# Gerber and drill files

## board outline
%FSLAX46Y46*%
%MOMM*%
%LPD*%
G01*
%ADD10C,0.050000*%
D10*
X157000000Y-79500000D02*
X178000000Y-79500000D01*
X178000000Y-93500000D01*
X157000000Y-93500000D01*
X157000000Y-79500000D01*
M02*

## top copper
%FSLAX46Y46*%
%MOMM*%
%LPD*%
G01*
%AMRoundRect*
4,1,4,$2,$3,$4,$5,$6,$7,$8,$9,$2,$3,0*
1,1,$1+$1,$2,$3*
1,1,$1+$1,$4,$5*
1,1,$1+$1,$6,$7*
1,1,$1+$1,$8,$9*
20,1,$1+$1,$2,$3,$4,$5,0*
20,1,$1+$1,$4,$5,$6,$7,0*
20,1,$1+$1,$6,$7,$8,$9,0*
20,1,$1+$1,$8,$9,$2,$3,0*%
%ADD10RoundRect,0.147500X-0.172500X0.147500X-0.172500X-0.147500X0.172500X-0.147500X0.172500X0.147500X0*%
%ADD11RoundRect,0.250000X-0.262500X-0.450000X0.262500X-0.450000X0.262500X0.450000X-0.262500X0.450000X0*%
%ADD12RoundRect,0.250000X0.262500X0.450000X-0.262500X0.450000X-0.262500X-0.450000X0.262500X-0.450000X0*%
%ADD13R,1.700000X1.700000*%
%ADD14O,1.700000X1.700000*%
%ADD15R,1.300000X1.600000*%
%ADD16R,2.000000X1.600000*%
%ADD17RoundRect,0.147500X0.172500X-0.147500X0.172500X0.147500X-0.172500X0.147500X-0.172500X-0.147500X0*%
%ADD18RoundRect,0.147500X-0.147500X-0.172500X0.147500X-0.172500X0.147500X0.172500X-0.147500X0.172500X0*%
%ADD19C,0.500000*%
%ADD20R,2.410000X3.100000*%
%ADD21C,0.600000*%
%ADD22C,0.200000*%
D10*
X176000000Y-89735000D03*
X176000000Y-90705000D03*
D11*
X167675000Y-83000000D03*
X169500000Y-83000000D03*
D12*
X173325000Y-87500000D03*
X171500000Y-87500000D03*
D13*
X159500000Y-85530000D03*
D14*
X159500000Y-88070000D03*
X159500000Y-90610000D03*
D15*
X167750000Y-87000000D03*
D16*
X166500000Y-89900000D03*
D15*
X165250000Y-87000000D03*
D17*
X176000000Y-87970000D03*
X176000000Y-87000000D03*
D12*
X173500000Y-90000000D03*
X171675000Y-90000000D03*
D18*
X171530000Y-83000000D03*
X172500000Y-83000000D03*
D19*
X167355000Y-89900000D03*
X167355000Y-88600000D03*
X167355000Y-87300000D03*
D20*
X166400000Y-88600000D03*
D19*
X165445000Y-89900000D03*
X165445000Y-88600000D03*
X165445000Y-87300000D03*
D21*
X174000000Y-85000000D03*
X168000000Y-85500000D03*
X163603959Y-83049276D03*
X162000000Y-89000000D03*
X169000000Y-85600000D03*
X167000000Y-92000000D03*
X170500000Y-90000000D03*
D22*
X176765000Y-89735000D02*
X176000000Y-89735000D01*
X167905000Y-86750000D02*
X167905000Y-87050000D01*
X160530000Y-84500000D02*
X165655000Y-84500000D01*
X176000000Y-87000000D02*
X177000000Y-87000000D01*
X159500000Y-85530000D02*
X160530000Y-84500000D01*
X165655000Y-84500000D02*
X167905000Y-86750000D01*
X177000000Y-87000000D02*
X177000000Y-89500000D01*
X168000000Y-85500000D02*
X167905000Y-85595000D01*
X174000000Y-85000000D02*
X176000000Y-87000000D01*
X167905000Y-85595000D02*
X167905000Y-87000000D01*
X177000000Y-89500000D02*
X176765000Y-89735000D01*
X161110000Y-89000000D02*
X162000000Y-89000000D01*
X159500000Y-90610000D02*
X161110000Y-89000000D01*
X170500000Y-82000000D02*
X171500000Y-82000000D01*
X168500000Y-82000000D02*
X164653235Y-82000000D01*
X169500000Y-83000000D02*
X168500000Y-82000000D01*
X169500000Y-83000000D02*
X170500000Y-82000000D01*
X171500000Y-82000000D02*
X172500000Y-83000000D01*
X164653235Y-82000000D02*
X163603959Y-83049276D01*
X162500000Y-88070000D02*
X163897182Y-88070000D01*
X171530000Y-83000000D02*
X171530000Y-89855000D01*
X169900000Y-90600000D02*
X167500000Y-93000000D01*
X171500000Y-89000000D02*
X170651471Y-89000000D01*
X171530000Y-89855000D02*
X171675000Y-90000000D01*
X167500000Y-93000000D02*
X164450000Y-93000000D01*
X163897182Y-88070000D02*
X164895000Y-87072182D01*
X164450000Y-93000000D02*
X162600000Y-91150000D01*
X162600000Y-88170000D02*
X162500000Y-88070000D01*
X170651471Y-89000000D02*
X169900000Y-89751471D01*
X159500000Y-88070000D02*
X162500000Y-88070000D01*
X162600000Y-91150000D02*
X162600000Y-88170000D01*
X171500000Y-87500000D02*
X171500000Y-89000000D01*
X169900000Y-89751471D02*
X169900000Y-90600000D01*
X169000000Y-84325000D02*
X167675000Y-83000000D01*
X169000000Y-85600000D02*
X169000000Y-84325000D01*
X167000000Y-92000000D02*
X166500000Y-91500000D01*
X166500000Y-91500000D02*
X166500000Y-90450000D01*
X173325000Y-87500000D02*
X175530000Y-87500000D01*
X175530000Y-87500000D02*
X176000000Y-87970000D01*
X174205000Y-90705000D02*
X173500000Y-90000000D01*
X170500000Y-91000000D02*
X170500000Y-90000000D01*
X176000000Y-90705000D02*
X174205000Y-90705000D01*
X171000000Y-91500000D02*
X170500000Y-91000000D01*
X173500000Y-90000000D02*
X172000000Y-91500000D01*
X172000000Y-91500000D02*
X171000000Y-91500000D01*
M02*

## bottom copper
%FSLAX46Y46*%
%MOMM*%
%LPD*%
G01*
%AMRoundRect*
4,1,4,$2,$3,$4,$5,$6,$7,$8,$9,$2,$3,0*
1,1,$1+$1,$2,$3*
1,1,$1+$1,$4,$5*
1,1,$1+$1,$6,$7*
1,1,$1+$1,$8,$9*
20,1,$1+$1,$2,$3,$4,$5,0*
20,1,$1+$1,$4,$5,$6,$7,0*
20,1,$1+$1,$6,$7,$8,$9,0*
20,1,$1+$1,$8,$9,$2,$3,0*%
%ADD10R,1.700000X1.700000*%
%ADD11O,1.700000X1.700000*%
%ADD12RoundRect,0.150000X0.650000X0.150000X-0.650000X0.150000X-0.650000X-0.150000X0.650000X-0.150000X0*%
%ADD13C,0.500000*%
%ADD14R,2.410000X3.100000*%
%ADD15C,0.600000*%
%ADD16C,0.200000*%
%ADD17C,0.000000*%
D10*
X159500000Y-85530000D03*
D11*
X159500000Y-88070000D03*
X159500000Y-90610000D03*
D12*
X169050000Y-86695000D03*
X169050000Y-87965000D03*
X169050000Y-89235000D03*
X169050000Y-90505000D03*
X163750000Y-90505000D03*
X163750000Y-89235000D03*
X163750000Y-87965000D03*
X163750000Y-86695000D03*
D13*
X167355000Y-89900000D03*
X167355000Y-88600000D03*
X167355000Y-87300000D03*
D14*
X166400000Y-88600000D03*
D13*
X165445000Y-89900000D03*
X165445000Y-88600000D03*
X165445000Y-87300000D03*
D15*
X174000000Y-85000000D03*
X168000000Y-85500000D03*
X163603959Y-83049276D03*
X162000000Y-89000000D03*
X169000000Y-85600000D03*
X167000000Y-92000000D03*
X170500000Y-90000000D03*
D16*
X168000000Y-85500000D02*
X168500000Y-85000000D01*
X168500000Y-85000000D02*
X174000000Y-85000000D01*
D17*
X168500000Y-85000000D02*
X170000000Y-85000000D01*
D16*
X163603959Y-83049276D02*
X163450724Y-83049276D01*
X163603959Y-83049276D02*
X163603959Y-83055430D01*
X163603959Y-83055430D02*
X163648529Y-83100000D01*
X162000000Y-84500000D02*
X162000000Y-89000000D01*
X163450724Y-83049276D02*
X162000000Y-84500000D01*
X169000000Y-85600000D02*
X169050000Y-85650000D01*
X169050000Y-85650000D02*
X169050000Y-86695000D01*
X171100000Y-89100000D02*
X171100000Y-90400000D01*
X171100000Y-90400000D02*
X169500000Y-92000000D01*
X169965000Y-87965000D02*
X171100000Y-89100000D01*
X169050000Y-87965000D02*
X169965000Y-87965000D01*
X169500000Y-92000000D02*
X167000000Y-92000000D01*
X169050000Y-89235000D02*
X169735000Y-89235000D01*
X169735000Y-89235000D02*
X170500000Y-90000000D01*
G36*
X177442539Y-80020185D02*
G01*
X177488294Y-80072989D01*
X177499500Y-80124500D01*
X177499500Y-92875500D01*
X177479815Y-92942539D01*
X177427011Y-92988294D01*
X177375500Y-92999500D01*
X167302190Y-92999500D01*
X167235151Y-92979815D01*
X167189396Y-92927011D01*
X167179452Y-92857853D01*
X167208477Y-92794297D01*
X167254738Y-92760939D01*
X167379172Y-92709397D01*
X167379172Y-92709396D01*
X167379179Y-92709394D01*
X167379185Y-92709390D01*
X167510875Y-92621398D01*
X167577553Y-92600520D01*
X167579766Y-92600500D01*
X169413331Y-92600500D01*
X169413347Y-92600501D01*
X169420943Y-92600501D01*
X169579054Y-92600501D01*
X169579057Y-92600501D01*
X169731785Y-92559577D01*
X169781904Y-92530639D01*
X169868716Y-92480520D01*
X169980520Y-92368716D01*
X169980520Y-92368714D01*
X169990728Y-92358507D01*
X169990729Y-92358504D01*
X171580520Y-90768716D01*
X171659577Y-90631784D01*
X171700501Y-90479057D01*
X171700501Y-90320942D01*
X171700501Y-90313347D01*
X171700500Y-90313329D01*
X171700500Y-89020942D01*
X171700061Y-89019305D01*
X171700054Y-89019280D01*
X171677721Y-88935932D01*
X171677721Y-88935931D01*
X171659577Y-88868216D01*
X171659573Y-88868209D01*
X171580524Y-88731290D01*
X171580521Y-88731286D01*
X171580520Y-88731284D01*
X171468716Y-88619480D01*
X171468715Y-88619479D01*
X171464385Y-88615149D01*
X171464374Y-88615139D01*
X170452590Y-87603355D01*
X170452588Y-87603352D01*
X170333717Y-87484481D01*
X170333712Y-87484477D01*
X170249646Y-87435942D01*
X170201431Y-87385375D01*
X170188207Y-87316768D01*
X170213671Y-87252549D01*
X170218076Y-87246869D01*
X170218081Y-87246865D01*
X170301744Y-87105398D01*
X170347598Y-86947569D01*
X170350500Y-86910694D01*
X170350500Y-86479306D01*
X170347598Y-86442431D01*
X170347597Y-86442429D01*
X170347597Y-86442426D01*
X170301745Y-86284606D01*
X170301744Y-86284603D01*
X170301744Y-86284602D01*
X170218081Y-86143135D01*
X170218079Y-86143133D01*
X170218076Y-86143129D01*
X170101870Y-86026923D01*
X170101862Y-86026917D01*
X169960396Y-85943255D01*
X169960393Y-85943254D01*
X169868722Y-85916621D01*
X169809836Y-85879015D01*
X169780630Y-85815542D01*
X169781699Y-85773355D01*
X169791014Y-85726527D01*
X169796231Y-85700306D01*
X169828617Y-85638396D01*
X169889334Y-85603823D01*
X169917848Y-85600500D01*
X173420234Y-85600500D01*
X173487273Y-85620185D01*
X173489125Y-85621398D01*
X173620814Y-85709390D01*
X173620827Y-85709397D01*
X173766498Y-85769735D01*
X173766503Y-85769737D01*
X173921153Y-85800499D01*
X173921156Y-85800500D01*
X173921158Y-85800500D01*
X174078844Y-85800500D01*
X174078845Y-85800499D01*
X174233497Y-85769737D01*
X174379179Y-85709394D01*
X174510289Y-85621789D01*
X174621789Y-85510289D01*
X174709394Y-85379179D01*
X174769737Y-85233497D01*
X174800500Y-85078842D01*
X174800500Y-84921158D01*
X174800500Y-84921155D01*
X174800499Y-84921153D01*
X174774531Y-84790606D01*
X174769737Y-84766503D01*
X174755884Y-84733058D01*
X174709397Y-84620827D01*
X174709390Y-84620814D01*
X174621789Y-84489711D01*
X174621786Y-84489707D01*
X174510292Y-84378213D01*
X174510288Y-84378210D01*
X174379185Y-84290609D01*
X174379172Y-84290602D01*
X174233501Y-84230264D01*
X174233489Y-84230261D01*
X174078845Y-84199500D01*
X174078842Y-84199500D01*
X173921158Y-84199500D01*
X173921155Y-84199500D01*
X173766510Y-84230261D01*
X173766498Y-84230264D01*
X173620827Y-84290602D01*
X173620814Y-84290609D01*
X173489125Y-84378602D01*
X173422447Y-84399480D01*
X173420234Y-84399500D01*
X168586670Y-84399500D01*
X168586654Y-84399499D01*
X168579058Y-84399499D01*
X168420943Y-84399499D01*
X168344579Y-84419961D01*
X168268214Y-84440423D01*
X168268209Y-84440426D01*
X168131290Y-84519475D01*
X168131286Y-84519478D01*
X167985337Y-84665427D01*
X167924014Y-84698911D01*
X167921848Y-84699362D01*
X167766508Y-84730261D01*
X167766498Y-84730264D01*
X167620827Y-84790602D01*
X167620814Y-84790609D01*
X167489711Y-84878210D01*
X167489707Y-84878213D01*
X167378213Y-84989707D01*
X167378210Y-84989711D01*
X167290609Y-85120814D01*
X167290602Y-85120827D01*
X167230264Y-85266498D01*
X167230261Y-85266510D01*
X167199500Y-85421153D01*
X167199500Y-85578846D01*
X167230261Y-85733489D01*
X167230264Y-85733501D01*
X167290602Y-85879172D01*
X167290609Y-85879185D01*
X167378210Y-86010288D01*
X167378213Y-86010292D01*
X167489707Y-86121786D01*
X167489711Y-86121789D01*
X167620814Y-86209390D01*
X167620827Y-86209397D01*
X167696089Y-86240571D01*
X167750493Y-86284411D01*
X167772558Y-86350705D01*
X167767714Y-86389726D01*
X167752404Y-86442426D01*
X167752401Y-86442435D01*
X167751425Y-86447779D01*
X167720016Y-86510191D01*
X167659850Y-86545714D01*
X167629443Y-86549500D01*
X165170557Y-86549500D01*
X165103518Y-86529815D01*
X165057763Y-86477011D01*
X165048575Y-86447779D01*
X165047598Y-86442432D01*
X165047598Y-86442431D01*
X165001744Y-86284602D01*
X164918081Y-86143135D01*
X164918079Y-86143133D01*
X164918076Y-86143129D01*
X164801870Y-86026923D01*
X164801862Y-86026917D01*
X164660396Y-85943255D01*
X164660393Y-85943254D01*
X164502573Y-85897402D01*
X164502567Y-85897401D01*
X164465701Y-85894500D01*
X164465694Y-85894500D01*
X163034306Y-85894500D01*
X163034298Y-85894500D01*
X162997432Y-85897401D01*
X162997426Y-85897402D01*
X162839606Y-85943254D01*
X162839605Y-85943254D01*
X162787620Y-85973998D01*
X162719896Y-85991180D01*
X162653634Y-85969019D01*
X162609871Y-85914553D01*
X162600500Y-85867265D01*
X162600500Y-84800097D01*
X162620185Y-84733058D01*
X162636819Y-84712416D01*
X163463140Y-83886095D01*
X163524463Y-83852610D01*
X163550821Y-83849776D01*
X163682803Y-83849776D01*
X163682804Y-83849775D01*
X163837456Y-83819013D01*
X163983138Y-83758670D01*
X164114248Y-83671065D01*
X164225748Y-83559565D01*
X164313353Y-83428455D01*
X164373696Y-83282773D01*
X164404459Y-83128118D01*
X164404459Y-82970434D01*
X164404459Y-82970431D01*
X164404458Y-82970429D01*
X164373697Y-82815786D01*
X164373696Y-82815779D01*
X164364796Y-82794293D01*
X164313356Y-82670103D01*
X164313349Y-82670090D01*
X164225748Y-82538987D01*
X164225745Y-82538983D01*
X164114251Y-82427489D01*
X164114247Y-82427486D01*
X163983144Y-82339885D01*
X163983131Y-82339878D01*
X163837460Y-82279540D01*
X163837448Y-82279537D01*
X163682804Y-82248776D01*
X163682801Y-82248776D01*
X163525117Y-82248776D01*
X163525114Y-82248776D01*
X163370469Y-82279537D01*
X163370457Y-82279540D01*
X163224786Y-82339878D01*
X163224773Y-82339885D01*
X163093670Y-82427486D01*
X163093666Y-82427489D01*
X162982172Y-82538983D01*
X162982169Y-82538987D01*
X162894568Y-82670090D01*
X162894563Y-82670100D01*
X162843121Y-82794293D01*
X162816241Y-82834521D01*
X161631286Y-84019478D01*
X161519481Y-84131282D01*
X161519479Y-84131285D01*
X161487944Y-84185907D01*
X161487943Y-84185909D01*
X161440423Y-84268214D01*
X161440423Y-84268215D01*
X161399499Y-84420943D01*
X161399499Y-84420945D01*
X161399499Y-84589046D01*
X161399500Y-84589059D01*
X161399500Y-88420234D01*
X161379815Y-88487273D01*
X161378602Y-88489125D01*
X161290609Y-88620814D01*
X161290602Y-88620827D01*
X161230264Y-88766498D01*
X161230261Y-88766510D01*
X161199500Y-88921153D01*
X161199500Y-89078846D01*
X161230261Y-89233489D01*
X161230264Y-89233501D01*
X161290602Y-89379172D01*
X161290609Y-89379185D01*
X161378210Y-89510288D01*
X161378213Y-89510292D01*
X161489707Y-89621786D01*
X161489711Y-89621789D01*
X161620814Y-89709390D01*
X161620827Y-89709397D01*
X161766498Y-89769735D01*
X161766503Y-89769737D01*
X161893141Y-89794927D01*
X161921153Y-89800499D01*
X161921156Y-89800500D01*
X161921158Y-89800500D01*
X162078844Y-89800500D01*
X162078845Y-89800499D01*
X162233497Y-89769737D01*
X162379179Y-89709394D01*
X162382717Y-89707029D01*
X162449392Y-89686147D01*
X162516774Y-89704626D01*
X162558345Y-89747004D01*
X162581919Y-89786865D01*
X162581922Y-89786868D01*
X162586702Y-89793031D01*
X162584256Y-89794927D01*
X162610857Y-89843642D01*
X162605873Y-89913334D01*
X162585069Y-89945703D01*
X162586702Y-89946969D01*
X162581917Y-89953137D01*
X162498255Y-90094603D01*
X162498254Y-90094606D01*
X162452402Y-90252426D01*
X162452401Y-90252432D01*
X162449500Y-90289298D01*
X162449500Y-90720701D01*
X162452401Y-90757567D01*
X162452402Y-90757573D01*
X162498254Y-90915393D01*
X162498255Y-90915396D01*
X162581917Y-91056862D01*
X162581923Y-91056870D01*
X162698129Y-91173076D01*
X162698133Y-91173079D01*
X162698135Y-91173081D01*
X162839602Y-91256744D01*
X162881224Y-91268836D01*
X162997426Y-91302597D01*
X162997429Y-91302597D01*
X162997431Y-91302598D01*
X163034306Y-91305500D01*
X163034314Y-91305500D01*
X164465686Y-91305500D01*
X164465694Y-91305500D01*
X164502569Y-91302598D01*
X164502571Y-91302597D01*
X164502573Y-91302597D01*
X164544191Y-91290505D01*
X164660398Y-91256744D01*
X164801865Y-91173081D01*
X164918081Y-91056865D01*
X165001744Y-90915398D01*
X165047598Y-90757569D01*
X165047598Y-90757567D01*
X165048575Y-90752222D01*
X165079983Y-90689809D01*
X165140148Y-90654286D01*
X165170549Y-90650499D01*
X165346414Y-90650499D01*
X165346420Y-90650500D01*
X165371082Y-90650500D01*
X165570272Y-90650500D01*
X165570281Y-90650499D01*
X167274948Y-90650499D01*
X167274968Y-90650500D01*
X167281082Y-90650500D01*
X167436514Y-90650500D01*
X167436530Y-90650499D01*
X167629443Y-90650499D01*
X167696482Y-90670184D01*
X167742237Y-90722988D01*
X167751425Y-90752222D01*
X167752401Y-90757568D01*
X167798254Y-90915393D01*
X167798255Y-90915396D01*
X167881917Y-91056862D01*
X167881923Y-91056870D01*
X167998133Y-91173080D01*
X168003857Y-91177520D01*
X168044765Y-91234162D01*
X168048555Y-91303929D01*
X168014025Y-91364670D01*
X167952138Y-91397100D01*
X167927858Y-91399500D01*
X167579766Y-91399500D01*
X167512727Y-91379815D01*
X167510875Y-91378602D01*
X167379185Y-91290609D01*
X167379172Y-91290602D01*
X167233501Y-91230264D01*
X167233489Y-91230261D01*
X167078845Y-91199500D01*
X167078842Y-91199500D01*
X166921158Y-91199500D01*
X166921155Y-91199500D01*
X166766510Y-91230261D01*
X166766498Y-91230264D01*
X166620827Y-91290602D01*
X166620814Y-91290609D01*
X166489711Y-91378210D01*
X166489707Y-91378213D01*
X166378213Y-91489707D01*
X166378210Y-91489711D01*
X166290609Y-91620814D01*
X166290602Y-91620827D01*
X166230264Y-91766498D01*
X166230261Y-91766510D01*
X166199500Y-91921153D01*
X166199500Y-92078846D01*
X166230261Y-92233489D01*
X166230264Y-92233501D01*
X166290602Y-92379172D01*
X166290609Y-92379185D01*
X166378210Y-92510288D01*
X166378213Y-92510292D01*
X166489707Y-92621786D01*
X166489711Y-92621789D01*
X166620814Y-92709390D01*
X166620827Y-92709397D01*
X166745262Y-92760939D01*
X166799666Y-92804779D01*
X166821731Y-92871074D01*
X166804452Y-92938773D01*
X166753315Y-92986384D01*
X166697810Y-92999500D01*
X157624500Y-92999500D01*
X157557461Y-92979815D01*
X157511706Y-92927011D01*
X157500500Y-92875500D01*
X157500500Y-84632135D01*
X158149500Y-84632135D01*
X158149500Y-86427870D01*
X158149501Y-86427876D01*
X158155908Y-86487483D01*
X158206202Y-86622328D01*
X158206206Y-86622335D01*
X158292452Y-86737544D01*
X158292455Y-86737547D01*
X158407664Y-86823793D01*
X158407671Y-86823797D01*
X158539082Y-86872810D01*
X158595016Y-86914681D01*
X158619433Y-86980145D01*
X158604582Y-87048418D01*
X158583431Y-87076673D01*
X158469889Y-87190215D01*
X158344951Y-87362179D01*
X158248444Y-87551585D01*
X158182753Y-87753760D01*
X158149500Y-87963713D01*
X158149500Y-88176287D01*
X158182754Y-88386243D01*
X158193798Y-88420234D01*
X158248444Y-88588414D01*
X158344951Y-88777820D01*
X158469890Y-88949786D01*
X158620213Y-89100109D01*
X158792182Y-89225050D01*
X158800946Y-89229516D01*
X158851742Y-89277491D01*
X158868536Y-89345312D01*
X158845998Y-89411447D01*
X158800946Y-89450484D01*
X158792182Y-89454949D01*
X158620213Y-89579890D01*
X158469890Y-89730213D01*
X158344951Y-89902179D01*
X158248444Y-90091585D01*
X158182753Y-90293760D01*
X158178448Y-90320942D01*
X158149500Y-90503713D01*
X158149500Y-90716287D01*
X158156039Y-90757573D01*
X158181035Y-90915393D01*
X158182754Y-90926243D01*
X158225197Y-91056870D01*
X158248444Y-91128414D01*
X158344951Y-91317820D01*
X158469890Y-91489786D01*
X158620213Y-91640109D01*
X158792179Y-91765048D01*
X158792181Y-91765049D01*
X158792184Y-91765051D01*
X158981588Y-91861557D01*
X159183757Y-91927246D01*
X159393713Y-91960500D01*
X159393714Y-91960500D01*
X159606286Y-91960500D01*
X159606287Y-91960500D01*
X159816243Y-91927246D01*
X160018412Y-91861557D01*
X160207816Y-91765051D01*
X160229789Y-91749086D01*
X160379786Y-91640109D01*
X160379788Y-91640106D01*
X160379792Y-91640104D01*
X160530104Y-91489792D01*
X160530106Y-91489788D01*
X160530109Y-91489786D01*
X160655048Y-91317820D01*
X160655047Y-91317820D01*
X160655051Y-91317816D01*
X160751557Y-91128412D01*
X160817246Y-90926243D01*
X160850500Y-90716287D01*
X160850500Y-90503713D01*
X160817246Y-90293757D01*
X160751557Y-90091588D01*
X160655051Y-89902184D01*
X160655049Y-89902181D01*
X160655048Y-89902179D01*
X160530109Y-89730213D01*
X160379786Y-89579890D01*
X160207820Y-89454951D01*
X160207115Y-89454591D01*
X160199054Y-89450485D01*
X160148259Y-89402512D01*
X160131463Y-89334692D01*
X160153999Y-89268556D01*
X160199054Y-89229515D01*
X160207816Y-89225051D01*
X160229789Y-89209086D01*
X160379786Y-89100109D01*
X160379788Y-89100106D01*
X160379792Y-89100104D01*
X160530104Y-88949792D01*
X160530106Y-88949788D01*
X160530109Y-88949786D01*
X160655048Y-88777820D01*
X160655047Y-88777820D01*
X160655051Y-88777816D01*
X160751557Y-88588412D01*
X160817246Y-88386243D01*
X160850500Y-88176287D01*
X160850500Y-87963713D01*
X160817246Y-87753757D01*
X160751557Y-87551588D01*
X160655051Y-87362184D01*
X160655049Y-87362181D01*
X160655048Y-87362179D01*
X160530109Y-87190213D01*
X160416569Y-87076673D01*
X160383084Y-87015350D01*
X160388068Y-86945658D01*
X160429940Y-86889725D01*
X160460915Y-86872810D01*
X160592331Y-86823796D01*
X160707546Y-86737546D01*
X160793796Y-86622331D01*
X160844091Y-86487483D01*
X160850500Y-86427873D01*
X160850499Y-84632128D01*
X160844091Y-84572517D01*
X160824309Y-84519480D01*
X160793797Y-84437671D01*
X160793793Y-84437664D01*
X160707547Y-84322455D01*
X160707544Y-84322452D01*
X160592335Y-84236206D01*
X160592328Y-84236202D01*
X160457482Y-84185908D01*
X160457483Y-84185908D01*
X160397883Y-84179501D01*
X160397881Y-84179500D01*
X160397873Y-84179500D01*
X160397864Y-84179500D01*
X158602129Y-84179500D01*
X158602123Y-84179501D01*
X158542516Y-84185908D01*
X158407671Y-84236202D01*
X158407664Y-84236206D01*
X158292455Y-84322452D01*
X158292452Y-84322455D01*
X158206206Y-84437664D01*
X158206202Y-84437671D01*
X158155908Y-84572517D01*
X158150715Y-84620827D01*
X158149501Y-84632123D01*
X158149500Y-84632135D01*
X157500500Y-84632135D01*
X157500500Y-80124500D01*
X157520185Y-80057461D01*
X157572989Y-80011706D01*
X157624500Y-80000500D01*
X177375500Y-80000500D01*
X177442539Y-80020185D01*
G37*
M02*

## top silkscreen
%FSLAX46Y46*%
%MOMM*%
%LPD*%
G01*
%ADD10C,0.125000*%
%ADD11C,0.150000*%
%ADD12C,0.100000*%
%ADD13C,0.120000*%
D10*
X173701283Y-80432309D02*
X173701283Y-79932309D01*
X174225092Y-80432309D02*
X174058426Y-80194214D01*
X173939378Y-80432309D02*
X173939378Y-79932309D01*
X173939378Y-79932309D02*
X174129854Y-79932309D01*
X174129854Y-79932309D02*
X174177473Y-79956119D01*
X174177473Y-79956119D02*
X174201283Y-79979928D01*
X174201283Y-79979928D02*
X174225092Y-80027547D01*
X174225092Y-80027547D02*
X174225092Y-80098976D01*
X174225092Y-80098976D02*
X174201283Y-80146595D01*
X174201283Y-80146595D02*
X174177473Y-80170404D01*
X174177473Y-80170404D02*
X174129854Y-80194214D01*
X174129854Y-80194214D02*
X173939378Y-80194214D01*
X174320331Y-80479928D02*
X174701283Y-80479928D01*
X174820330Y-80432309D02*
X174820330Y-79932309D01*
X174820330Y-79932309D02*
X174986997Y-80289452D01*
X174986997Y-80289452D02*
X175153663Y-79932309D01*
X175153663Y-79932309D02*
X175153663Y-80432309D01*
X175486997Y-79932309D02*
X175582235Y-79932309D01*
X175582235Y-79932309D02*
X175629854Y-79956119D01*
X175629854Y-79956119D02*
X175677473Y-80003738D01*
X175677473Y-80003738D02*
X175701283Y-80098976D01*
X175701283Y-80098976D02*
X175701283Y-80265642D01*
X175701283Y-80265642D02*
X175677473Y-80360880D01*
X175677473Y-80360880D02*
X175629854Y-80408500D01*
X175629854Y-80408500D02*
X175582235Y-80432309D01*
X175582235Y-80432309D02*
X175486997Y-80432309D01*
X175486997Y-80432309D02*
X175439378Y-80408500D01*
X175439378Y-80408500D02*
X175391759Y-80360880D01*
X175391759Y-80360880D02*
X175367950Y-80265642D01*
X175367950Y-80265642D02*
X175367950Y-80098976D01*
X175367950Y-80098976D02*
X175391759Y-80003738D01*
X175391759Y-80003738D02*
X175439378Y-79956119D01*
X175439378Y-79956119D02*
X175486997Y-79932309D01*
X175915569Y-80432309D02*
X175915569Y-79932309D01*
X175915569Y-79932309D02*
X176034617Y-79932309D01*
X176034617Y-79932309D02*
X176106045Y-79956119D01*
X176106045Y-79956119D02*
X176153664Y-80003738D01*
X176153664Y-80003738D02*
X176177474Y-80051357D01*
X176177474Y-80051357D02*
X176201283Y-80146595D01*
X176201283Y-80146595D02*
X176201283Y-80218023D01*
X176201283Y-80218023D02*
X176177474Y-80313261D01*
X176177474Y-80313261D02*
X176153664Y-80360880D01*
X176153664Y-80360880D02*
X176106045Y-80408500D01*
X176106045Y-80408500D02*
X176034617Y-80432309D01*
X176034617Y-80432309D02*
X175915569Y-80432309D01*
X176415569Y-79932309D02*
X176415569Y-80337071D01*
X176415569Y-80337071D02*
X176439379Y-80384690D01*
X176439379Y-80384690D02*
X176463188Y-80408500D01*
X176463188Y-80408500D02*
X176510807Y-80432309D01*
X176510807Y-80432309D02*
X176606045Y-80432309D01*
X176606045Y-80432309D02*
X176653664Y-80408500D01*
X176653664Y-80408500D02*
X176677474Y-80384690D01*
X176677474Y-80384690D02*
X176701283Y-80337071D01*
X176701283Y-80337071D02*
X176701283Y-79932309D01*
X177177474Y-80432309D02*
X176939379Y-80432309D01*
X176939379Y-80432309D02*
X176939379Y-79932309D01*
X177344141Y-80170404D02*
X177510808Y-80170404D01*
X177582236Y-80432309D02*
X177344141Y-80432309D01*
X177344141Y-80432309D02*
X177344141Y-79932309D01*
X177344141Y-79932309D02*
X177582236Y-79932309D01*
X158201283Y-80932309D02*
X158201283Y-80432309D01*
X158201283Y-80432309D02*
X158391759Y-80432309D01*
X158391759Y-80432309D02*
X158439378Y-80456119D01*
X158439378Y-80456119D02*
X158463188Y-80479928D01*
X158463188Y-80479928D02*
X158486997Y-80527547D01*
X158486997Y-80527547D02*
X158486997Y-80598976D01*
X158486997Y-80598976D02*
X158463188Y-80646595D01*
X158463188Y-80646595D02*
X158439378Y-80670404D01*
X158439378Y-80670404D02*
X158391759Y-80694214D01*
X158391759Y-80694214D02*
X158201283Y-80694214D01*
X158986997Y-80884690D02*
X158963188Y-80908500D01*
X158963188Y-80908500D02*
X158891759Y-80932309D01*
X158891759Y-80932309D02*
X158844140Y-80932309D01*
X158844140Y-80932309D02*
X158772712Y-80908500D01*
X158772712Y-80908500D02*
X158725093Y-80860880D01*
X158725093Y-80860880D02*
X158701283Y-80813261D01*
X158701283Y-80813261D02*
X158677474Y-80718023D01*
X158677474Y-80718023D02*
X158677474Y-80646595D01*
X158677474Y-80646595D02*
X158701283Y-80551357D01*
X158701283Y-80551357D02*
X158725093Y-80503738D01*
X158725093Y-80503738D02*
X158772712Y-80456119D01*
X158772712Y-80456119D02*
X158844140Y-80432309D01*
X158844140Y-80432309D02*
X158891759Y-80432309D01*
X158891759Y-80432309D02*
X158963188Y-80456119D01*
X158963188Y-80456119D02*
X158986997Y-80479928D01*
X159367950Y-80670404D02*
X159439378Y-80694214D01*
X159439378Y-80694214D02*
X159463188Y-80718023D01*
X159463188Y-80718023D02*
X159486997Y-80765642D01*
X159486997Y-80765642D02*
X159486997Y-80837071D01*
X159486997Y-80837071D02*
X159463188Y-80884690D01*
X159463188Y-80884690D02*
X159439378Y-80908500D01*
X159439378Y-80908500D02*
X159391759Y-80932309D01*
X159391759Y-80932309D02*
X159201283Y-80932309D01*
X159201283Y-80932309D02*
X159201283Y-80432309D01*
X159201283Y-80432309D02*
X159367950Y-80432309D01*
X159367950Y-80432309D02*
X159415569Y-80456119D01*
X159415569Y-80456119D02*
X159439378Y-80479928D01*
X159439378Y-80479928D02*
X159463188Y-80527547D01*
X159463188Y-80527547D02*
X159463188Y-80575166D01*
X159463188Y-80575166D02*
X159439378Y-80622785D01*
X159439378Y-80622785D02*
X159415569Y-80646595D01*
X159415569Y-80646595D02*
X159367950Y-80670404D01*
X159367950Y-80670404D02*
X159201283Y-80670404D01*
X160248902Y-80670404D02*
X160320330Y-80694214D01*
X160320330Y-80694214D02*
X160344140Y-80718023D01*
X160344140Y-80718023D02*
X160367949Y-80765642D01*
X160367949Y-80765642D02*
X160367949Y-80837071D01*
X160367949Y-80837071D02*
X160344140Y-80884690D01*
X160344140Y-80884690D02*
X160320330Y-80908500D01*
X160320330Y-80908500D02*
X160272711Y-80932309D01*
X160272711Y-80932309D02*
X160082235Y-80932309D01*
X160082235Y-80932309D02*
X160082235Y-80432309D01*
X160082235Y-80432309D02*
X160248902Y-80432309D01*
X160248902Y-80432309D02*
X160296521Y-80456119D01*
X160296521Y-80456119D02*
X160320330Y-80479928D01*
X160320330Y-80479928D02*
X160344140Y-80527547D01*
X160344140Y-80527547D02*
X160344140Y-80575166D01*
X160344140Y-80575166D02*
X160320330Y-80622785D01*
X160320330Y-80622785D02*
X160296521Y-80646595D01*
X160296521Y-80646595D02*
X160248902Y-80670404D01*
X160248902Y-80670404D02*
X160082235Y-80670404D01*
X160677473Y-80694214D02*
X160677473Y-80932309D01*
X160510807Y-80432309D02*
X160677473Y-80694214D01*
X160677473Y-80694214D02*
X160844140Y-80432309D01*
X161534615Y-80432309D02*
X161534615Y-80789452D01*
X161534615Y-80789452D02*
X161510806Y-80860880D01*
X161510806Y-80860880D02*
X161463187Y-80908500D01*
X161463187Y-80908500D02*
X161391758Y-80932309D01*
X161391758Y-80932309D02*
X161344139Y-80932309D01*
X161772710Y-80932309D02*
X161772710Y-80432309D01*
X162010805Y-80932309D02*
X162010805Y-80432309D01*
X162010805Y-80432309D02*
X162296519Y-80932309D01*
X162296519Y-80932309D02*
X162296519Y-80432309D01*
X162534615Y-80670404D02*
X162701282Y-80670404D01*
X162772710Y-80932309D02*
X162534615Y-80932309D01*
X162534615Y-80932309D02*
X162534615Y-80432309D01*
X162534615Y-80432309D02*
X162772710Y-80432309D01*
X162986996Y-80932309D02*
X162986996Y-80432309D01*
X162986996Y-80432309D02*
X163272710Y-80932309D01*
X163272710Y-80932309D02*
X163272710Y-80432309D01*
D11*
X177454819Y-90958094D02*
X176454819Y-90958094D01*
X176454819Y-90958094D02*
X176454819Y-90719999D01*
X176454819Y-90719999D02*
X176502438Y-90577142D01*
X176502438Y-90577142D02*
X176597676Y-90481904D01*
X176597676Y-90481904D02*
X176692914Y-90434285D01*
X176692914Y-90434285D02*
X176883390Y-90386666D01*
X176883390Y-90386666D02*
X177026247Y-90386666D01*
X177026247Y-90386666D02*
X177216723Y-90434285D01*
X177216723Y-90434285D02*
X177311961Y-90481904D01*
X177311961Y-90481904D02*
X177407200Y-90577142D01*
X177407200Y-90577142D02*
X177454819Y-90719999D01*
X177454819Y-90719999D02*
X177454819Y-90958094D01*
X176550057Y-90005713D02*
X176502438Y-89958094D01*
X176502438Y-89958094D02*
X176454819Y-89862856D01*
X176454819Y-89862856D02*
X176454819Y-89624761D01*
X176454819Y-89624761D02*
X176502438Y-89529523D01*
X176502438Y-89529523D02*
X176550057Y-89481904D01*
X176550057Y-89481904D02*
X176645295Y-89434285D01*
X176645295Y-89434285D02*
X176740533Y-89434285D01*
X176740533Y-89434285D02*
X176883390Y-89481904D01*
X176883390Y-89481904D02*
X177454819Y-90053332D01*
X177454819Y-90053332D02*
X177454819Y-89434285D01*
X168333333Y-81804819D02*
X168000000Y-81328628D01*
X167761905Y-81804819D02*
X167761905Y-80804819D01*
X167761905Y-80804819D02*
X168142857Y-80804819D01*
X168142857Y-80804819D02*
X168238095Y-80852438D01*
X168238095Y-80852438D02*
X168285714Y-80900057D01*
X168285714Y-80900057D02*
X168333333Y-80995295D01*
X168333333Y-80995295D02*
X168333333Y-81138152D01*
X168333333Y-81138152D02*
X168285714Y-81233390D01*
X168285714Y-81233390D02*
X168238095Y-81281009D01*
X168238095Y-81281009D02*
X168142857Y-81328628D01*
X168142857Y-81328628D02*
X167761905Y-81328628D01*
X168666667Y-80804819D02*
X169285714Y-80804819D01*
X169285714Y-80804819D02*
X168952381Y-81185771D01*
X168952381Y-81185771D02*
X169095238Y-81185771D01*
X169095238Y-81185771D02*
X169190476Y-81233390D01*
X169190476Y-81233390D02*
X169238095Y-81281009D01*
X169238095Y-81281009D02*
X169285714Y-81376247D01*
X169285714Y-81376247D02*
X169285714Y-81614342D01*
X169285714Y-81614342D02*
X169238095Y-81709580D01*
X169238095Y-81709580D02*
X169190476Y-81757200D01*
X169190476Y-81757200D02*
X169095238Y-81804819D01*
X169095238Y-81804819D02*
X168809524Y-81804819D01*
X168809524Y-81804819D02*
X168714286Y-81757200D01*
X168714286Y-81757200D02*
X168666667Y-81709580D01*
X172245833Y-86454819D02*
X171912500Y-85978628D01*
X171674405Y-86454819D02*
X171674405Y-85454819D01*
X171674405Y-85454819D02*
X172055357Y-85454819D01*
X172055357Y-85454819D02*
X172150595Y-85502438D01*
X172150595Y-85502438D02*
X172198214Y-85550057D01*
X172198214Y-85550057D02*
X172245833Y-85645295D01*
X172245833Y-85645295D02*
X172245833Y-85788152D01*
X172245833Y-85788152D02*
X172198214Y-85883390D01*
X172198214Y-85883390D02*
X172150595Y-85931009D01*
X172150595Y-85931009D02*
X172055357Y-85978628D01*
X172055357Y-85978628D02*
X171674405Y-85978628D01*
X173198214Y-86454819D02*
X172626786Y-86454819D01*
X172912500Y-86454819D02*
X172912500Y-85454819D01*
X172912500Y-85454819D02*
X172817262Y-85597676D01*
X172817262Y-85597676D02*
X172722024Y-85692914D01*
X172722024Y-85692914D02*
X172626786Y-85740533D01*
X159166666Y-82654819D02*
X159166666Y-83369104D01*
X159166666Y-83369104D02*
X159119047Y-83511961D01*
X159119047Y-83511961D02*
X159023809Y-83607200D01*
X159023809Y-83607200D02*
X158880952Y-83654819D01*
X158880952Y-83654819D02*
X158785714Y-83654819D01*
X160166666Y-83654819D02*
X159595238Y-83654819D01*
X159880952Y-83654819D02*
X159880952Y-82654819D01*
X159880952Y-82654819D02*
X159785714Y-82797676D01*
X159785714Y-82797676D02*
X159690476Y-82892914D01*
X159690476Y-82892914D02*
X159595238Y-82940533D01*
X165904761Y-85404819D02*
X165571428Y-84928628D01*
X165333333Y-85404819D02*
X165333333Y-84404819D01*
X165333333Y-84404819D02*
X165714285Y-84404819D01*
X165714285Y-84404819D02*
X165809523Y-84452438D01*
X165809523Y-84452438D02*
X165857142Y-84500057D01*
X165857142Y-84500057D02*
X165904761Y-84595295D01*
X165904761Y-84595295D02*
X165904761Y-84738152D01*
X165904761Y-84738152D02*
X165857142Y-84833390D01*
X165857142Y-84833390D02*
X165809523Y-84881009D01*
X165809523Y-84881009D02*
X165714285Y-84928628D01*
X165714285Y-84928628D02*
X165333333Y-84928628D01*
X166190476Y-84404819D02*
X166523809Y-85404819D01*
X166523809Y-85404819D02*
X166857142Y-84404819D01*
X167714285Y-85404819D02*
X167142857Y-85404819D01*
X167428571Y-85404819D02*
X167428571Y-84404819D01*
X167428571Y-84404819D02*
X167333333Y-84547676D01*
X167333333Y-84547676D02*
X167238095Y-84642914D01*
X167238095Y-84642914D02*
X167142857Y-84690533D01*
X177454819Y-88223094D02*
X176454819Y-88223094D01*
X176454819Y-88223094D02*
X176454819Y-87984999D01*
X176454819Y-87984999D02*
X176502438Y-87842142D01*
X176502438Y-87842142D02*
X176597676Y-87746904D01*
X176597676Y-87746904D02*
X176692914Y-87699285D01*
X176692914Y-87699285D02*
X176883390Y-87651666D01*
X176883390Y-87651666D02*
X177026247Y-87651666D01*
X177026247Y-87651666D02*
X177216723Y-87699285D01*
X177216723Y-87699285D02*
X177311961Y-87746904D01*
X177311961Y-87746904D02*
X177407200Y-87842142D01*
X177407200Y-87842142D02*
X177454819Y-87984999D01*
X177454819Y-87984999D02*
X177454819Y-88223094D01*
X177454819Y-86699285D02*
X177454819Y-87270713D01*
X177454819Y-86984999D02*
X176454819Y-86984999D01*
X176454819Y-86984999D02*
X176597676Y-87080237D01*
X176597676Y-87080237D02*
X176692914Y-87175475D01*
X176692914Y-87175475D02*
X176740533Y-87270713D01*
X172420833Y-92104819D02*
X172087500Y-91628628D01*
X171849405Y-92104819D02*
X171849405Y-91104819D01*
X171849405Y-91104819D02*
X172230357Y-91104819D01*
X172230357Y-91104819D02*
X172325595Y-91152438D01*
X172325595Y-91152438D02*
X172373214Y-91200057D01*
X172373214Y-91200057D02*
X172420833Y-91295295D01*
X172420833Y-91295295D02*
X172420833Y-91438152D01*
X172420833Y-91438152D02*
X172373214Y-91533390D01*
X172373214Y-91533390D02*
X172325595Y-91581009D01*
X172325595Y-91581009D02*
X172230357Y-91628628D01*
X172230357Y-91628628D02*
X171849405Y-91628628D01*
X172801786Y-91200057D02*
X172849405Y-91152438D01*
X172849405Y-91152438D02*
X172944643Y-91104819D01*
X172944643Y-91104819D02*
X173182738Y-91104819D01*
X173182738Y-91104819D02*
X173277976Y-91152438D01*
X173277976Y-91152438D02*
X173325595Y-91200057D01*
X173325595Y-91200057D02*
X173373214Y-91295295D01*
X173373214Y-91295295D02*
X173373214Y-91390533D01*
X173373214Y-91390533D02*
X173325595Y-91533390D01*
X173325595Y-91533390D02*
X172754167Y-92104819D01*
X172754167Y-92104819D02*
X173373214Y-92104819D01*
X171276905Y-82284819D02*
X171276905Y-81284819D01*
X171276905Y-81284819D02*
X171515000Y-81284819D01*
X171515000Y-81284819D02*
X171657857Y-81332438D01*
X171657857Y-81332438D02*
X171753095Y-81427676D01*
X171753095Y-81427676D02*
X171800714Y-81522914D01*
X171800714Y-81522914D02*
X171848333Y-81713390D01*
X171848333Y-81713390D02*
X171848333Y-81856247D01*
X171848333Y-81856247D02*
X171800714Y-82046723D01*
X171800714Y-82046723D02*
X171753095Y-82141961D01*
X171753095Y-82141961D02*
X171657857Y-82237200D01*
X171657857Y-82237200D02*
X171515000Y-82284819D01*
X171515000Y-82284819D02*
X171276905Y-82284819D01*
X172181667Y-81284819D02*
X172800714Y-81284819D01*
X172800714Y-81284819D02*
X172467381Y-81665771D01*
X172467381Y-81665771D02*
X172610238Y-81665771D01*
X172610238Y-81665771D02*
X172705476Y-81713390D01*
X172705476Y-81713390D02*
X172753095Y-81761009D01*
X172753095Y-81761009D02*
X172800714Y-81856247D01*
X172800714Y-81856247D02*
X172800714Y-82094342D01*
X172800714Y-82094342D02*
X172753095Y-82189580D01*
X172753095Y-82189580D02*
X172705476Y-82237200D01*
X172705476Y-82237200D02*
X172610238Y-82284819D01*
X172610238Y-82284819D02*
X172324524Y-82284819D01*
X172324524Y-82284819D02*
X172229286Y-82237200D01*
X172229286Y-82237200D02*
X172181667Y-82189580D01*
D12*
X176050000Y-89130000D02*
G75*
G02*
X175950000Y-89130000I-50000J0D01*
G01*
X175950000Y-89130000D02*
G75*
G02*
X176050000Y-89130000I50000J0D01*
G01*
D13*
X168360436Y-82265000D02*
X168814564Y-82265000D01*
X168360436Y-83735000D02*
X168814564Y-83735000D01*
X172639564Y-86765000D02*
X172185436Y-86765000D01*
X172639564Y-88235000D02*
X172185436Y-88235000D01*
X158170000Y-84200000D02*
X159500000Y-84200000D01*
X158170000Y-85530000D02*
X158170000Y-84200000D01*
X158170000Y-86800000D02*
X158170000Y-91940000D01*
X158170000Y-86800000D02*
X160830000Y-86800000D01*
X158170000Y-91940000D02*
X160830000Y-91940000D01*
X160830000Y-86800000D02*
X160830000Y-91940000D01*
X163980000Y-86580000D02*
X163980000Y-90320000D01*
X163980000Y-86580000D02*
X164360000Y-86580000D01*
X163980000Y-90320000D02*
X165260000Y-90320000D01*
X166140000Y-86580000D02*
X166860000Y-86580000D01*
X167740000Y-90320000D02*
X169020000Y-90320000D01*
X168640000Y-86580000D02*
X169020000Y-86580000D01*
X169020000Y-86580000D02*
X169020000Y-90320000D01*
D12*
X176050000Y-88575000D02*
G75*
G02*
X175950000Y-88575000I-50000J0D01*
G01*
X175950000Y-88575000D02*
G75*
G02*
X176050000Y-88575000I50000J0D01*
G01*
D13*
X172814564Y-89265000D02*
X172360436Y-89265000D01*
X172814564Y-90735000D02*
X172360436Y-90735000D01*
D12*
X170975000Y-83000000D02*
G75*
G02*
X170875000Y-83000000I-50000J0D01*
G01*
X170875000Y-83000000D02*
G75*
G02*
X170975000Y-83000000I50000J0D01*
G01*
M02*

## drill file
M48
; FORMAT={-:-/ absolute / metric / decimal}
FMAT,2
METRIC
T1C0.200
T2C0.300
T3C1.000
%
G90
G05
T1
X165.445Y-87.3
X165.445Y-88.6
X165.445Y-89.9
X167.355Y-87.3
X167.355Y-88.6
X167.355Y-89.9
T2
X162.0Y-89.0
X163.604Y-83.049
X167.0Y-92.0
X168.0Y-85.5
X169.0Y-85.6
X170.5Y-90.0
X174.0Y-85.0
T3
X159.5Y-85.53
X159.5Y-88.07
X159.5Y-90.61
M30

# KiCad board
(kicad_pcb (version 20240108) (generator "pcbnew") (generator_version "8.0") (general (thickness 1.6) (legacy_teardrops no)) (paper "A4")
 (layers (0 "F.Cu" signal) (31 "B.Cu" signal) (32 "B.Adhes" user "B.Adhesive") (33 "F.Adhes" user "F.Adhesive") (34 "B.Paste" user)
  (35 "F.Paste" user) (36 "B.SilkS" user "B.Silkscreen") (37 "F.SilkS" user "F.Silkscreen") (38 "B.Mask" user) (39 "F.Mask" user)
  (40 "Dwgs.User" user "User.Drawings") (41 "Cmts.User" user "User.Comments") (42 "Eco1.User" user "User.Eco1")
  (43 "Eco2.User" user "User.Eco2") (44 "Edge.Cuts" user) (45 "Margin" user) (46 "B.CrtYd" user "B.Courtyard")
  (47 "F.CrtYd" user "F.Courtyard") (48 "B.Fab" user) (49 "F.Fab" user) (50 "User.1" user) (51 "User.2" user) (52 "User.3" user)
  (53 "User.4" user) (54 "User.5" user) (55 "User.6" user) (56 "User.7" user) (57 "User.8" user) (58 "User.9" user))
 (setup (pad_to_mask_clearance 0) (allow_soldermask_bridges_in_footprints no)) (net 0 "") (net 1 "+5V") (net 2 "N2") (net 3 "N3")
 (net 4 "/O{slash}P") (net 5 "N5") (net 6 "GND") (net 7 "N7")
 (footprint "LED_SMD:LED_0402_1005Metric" (layer "F.Cu") (at 176 90.22 -90)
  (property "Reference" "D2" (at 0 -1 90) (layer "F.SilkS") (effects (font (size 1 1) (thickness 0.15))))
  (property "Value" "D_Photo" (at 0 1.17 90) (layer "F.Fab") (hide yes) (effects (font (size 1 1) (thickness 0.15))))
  (fp_circle (center -1.09 0) (end -1.04 0) (stroke (width 0.1) (type solid)) (fill none) (layer "F.SilkS"))
  (pad "1" smd roundrect (at -0.485 0 270) (size 0.59 0.64) (layers "F.Cu" "F.Paste" "F.Mask") (roundrect_rratio 0.25) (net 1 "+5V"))
  (pad "2" smd roundrect (at 0.485 0 270) (size 0.59 0.64) (layers "F.Cu" "F.Paste" "F.Mask") (roundrect_rratio 0.25) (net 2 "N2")))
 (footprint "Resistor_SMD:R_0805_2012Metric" (layer "F.Cu") (at 168.5875 83)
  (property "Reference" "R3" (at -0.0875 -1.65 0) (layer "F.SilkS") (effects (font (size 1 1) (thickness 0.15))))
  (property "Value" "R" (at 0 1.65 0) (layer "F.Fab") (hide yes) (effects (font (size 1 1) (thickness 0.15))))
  (fp_line (start -0.227064 -0.735) (end 0.227064 -0.735) (stroke (width 0.12) (type solid)) (layer "F.SilkS"))
  (fp_line (start -0.227064 0.735) (end 0.227064 0.735) (stroke (width 0.12) (type solid)) (layer "F.SilkS"))
  (pad "1" smd roundrect (at -0.9125 0) (size 1.025 1.4) (layers "F.Cu" "F.Paste" "F.Mask") (roundrect_rratio 0.243902) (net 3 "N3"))
  (pad "2" smd roundrect (at 0.9125 0) (size 1.025 1.4) (layers "F.Cu" "F.Paste" "F.Mask") (roundrect_rratio 0.243902) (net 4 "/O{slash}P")))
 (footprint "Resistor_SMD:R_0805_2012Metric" (layer "F.Cu") (at 172.4125 87.5 180)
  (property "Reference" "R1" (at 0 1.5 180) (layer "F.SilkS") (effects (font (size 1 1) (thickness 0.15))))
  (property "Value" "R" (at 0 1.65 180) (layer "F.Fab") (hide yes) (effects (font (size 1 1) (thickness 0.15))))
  (fp_line (start -0.227064 0.735) (end 0.227064 0.735) (stroke (width 0.12) (type solid)) (layer "F.SilkS"))
  (fp_line (start -0.227064 -0.735) (end 0.227064 -0.735) (stroke (width 0.12) (type solid)) (layer "F.SilkS"))
  (pad "1" smd roundrect (at -0.9125 0 180) (size 1.025 1.4) (layers "F.Cu" "F.Paste" "F.Mask") (roundrect_rratio 0.243902) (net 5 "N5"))
  (pad "2" smd roundrect (at 0.9125 0 180) (size 1.025 1.4) (layers "F.Cu" "F.Paste" "F.Mask") (roundrect_rratio 0.243902) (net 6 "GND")))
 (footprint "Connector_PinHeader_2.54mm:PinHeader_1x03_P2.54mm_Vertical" (layer "F.Cu") (at 159.5 85.53)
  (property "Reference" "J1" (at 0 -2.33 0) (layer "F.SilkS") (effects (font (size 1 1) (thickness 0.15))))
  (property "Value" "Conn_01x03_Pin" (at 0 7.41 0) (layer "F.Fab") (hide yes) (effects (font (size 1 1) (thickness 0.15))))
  (fp_line (start -1.33 -1.33) (end 0 -1.33) (stroke (width 0.12) (type solid)) (layer "F.SilkS"))
  (fp_line (start -1.33 0) (end -1.33 -1.33) (stroke (width 0.12) (type solid)) (layer "F.SilkS"))
  (fp_line (start -1.33 1.27) (end -1.33 6.41) (stroke (width 0.12) (type solid)) (layer "F.SilkS"))
  (fp_line (start -1.33 1.27) (end 1.33 1.27) (stroke (width 0.12) (type solid)) (layer "F.SilkS"))
  (fp_line (start -1.33 6.41) (end 1.33 6.41) (stroke (width 0.12) (type solid)) (layer "F.SilkS"))
  (fp_line (start 1.33 1.27) (end 1.33 6.41) (stroke (width 0.12) (type solid)) (layer "F.SilkS"))
  (pad "1" thru_hole rect (at 0 0) (size 1.7 1.7) (drill 1) (layers "*.Cu" "*.Mask") (remove_unused_layers no) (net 1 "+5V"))
  (pad "2" thru_hole oval (at 0 2.54) (size 1.7 1.7) (drill 1) (layers "*.Cu" "*.Mask") (remove_unused_layers no) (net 6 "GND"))
  (pad "3" thru_hole oval (at 0 5.08) (size 1.7 1.7) (drill 1) (layers "*.Cu" "*.Mask") (remove_unused_layers no) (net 4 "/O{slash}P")))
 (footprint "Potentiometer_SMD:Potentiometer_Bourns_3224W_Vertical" (layer "F.Cu") (at 166.5 88.45)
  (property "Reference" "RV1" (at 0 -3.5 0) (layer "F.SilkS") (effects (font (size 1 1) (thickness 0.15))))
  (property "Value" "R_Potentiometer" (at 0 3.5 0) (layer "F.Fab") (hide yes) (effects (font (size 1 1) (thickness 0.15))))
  (fp_line (start -2.52 -1.87) (end -2.52 1.87) (stroke (width 0.12) (type solid)) (layer "F.SilkS"))
  (fp_line (start -2.52 -1.87) (end -2.14 -1.87) (stroke (width 0.12) (type solid)) (layer "F.SilkS"))
  (fp_line (start -2.52 1.87) (end -1.24 1.87) (stroke (width 0.12) (type solid)) (layer "F.SilkS"))
  (fp_line (start -0.36 -1.87) (end 0.36 -1.87) (stroke (width 0.12) (type solid)) (layer "F.SilkS"))
  (fp_line (start 1.24 1.87) (end 2.52 1.87) (stroke (width 0.12) (type solid)) (layer "F.SilkS"))
  (fp_line (start 2.14 -1.87) (end 2.52 -1.87) (stroke (width 0.12) (type solid)) (layer "F.SilkS"))
  (fp_line (start 2.52 -1.87) (end 2.52 1.87) (stroke (width 0.12) (type solid)) (layer "F.SilkS"))
  (pad "1" smd rect (at 1.25 -1.45) (size 1.3 1.6) (layers "F.Cu" "F.Paste" "F.Mask") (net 1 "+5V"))
  (pad "2" smd rect (at 0 1.45) (size 2 1.6) (layers "F.Cu" "F.Paste" "F.Mask") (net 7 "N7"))
  (pad "3" smd rect (at -1.25 -1.45) (size 1.3 1.6) (layers "F.Cu" "F.Paste" "F.Mask") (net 6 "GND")))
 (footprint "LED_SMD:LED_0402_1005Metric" (layer "F.Cu") (at 176 87.485 90)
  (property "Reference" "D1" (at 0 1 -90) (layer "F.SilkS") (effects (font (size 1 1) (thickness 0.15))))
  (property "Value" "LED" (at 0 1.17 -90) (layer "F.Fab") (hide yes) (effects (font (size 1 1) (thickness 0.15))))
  (fp_circle (center -1.09 0) (end -1.04 0) (stroke (width 0.1) (type solid)) (fill none) (layer "F.SilkS"))
  (pad "1" smd roundrect (at -0.485 0 90) (size 0.59 0.64) (layers "F.Cu" "F.Paste" "F.Mask") (roundrect_rratio 0.25) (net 5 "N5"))
  (pad "2" smd roundrect (at 0.485 0 90) (size 0.59 0.64) (layers "F.Cu" "F.Paste" "F.Mask") (roundrect_rratio 0.25) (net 1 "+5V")))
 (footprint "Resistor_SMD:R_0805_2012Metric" (layer "F.Cu") (at 172.5875 90 180)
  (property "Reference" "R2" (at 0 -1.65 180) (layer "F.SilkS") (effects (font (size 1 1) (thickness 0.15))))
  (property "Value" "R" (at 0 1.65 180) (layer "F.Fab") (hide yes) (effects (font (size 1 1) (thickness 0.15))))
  (fp_line (start -0.227064 0.735) (end 0.227064 0.735) (stroke (width 0.12) (type solid)) (layer "F.SilkS"))
  (fp_line (start -0.227064 -0.735) (end 0.227064 -0.735) (stroke (width 0.12) (type solid)) (layer "F.SilkS"))
  (pad "1" smd roundrect (at -0.9125 0 180) (size 1.025 1.4) (layers "F.Cu" "F.Paste" "F.Mask") (roundrect_rratio 0.243902) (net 2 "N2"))
  (pad "2" smd roundrect (at 0.9125 0 180) (size 1.025 1.4) (layers "F.Cu" "F.Paste" "F.Mask") (roundrect_rratio 0.243902) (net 6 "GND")))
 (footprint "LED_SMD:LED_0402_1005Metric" (layer "F.Cu") (at 172.015 83)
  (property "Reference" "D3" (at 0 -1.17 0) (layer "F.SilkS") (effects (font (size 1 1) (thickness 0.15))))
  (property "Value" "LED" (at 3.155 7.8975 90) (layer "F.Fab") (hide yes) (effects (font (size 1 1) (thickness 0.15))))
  (fp_circle (center -1.09 0) (end -1.04 0) (stroke (width 0.1) (type solid)) (fill none) (layer "F.SilkS"))
  (pad "1" smd roundrect (at -0.485 0) (size 0.59 0.64) (layers "F.Cu" "F.Paste" "F.Mask") (roundrect_rratio 0.25) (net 6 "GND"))
  (pad "2" smd roundrect (at 0.485 0) (size 0.59 0.64) (layers "F.Cu" "F.Paste" "F.Mask") (roundrect_rratio 0.25) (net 4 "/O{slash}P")))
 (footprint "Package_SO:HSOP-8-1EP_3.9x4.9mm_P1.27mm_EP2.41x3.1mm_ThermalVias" (layer "B.Cu") (at 166.4 88.6 180)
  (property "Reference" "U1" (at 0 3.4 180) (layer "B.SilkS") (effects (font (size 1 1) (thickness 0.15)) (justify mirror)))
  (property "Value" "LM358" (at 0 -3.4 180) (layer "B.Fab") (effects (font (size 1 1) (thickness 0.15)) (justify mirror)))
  (pad "" smd roundrect (at -0.6 -0.775 180) (size 0.97 1.25) (layers "B.Paste") (roundrect_rratio 0.25))
  (pad "" smd roundrect (at -0.6 0.775 180) (size 0.97 1.25) (layers "B.Paste") (roundrect_rratio 0.25))
  (pad "" smd roundrect (at 0.6 -0.775 180) (size 0.97 1.25) (layers "B.Paste") (roundrect_rratio 0.25))
  (pad "" smd roundrect (at 0.6 0.775 180) (size 0.97 1.25) (layers "B.Paste") (roundrect_rratio 0.25))
  (pad "1" smd roundrect (at -2.65 1.905 180) (size 1.6 0.6) (layers "B.Cu" "B.Paste" "B.Mask") (roundrect_rratio 0.25) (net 3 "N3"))
  (pad "2" smd roundrect (at -2.65 0.635 180) (size 1.6 0.6) (layers "B.Cu" "B.Paste" "B.Mask") (roundrect_rratio 0.25) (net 7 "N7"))
  (pad "3" smd roundrect (at -2.65 -0.635 180) (size 1.6 0.6) (layers "B.Cu" "B.Paste" "B.Mask") (roundrect_rratio 0.25) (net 2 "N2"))
  (pad "4" smd roundrect (at -2.65 -1.905 180) (size 1.6 0.6) (layers "B.Cu" "B.Paste" "B.Mask") (roundrect_rratio 0.25))
  (pad "5" smd roundrect (at 2.65 -1.905 180) (size 1.6 0.6) (layers "B.Cu" "B.Paste" "B.Mask") (roundrect_rratio 0.25))
  (pad "6" smd roundrect (at 2.65 -0.635 180) (size 1.6 0.6) (layers "B.Cu" "B.Paste" "B.Mask") (roundrect_rratio 0.25))
  (pad "7" smd roundrect (at 2.65 0.635 180) (size 1.6 0.6) (layers "B.Cu" "B.Paste" "B.Mask") (roundrect_rratio 0.25))
  (pad "8" smd roundrect (at 2.65 1.905 180) (size 1.6 0.6) (layers "B.Cu" "B.Paste" "B.Mask") (roundrect_rratio 0.25))
  (pad "9" thru_hole circle (at -0.955 -1.3 180) (size 0.5 0.5) (drill 0.2) (layers "*.Cu") (remove_unused_layers no))
  (pad "9" thru_hole circle (at -0.955 0 180) (size 0.5 0.5) (drill 0.2) (layers "*.Cu") (remove_unused_layers no))
  (pad "9" thru_hole circle (at -0.955 1.3 180) (size 0.5 0.5) (drill 0.2) (layers "*.Cu") (remove_unused_layers no))
  (pad "9" smd rect (at 0 0 180) (size 2.41 3.1) (layers "F.Cu") (zone_connect 2))
  (pad "9" smd rect (at 0 0 180) (size 2.41 3.1) (layers "B.Cu" "B.Mask") (zone_connect 2))
  (pad "9" thru_hole circle (at 0.955 -1.3 180) (size 0.5 0.5) (drill 0.2) (layers "*.Cu") (remove_unused_layers no))
  (pad "9" thru_hole circle (at 0.955 0 180) (size 0.5 0.5) (drill 0.2) (layers "*.Cu") (remove_unused_layers no))
  (pad "9" thru_hole circle (at 0.955 1.3 180) (size 0.5 0.5) (drill 0.2) (layers "*.Cu") (remove_unused_layers no)))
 (gr_rect (start 157 79.5) (end 178 93.5) (stroke (width 0.05) (type default)) (fill none) (layer "Edge.Cuts"))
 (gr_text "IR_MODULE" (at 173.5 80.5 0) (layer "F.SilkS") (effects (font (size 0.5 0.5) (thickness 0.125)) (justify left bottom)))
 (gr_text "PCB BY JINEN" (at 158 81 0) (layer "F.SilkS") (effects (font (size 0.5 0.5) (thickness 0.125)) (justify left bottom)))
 (segment (start 176.765 89.735) (end 176 89.735) (width 0.2) (layer "F.Cu") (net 1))
 (segment (start 167.905 86.75) (end 167.905 87.05) (width 0.2) (layer "F.Cu") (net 1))
 (segment (start 160.53 84.5) (end 165.655 84.5) (width 0.2) (layer "F.Cu") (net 1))
 (segment (start 176 87) (end 177 87) (width 0.2) (layer "F.Cu") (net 1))
 (segment (start 159.5 85.53) (end 160.53 84.5) (width 0.2) (layer "F.Cu") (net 1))
 (segment (start 165.655 84.5) (end 167.905 86.75) (width 0.2) (layer "F.Cu") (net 1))
 (segment (start 177 87) (end 177 89.5) (width 0.2) (layer "F.Cu") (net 1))
 (segment (start 168 85.5) (end 167.905 85.595) (width 0.2) (layer "F.Cu") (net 1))
 (segment (start 174 85) (end 176 87) (width 0.2) (layer "F.Cu") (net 1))
 (segment (start 167.905 85.595) (end 167.905 87) (width 0.2) (layer "F.Cu") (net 1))
 (segment (start 177 89.5) (end 176.765 89.735) (width 0.2) (layer "F.Cu") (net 1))
 (via (at 174 85) (size 0.6) (drill 0.3) (layers "F.Cu" "B.Cu") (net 1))
 (via (at 168 85.5) (size 0.6) (drill 0.3) (layers "F.Cu" "B.Cu") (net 1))
 (segment (start 168 85.5) (end 168.5 85) (width 0.2) (layer "B.Cu") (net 1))
 (segment (start 168.5 85) (end 174 85) (width 0.2) (layer "B.Cu") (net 1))
 (segment (start 168.5 85) (end 170 85) (width 0) (layer "B.Cu") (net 1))
 (segment (start 161.11 89) (end 162 89) (width 0.2) (layer "F.Cu") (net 4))
 (segment (start 159.5 90.61) (end 161.11 89) (width 0.2) (layer "F.Cu") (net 4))
 (segment (start 170.5 82) (end 171.5 82) (width 0.2) (layer "F.Cu") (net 4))
 (segment (start 168.5 82) (end 164.653235 82) (width 0.2) (layer "F.Cu") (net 4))
 (segment (start 169.5 83) (end 168.5 82) (width 0.2) (layer "F.Cu") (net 4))
 (segment (start 169.5 83) (end 170.5 82) (width 0.2) (layer "F.Cu") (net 4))
 (segment (start 171.5 82) (end 172.5 83) (width 0.2) (layer "F.Cu") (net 4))
 (segment (start 164.653235 82) (end 163.603959 83.049276) (width 0.2) (layer "F.Cu") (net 4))
 (via (at 163.603959 83.049276) (size 0.6) (drill 0.3) (layers "F.Cu" "B.Cu") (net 4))
 (via (at 162 89) (size 0.6) (drill 0.3) (layers "F.Cu" "B.Cu") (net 4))
 (segment (start 163.603959 83.049276) (end 163.450724 83.049276) (width 0.2) (layer "B.Cu") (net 4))
 (segment (start 163.603959 83.049276) (end 163.603959 83.05543) (width 0.2) (layer "B.Cu") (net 4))
 (segment (start 163.603959 83.05543) (end 163.648529 83.1) (width 0.2) (layer "B.Cu") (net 4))
 (segment (start 162 84.5) (end 162 89) (width 0.2) (layer "B.Cu") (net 4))
 (segment (start 163.450724 83.049276) (end 162 84.5) (width 0.2) (layer "B.Cu") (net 4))
 (segment (start 162.5 88.07) (end 163.897182 88.07) (width 0.2) (layer "F.Cu") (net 6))
 (segment (start 171.53 83) (end 171.53 89.855) (width 0.2) (layer "F.Cu") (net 6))
 (segment (start 169.9 90.6) (end 167.5 93) (width 0.2) (layer "F.Cu") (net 6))
 (segment (start 171.5 89) (end 170.651471 89) (width 0.2) (layer "F.Cu") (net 6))
 (segment (start 171.53 89.855) (end 171.675 90) (width 0.2) (layer "F.Cu") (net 6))
 (segment (start 167.5 93) (end 164.45 93) (width 0.2) (layer "F.Cu") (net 6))
 (segment (start 163.897182 88.07) (end 164.895 87.072182) (width 0.2) (layer "F.Cu") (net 6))
 (segment (start 164.45 93) (end 162.6 91.15) (width 0.2) (layer "F.Cu") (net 6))
 (segment (start 162.6 88.17) (end 162.5 88.07) (width 0.2) (layer "F.Cu") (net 6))
 (segment (start 170.651471 89) (end 169.9 89.751471) (width 0.2) (layer "F.Cu") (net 6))
 (segment (start 159.5 88.07) (end 162.5 88.07) (width 0.2) (layer "F.Cu") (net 6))
 (segment (start 162.6 91.15) (end 162.6 88.17) (width 0.2) (layer "F.Cu") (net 6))
 (segment (start 171.5 87.5) (end 171.5 89) (width 0.2) (layer "F.Cu") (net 6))
 (segment (start 169.9 89.751471) (end 169.9 90.6) (width 0.2) (layer "F.Cu") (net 6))
 (segment (start 169 84.325) (end 167.675 83) (width 0.2) (layer "F.Cu") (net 3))
 (segment (start 169 85.6) (end 169 84.325) (width 0.2) (layer "F.Cu") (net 3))
 (via (at 169 85.6) (size 0.6) (drill 0.3) (layers "F.Cu" "B.Cu") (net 3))
 (segment (start 169 85.6) (end 169.05 85.65) (width 0.2) (layer "B.Cu") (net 3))
 (segment (start 169.05 85.65) (end 169.05 86.695) (width 0.2) (layer "B.Cu") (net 3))
 (segment (start 167 92) (end 166.5 91.5) (width 0.2) (layer "F.Cu") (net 7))
 (segment (start 166.5 91.5) (end 166.5 90.45) (width 0.2) (layer "F.Cu") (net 7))
 (via (at 167 92) (size 0.6) (drill 0.3) (layers "F.Cu" "B.Cu") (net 7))
 (segment (start 171.1 89.1) (end 171.1 90.4) (width 0.2) (layer "B.Cu") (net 7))
 (segment (start 171.1 90.4) (end 169.5 92) (width 0.2) (layer "B.Cu") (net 7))
 (segment (start 169.965 87.965) (end 171.1 89.1) (width 0.2) (layer "B.Cu") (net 7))
 (segment (start 169.05 87.965) (end 169.965 87.965) (width 0.2) (layer "B.Cu") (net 7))
 (segment (start 169.5 92) (end 167 92) (width 0.2) (layer "B.Cu") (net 7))
 (segment (start 173.325 87.5) (end 175.53 87.5) (width 0.2) (layer "F.Cu") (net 5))
 (segment (start 175.53 87.5) (end 176 87.97) (width 0.2) (layer "F.Cu") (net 5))
 (segment (start 174.205 90.705) (end 173.5 90) (width 0.2) (layer "F.Cu") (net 2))
 (segment (start 170.5 91) (end 170.5 90) (width 0.2) (layer "F.Cu") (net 2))
 (segment (start 176 90.705) (end 174.205 90.705) (width 0.2) (layer "F.Cu") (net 2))
 (segment (start 171 91.5) (end 170.5 91) (width 0.2) (layer "F.Cu") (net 2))
 (segment (start 173.5 90) (end 172 91.5) (width 0.2) (layer "F.Cu") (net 2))
 (segment (start 172 91.5) (end 171 91.5) (width 0.2) (layer "F.Cu") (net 2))
 (via (at 170.5 90) (size 0.6) (drill 0.3) (layers "F.Cu" "B.Cu") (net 2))
 (segment (start 169.05 89.235) (end 169.735 89.235) (width 0.2) (layer "B.Cu") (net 2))
 (segment (start 169.735 89.235) (end 170.5 90) (width 0.2) (layer "B.Cu") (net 2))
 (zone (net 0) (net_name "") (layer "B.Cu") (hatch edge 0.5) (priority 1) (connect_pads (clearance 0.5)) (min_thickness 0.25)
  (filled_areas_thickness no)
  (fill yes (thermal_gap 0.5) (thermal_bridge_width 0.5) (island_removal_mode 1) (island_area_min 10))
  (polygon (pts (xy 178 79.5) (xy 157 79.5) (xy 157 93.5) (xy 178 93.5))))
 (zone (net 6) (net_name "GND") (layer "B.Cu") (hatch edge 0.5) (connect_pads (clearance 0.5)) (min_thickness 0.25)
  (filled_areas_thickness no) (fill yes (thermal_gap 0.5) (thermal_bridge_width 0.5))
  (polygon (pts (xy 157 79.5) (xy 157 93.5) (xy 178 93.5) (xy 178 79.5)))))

